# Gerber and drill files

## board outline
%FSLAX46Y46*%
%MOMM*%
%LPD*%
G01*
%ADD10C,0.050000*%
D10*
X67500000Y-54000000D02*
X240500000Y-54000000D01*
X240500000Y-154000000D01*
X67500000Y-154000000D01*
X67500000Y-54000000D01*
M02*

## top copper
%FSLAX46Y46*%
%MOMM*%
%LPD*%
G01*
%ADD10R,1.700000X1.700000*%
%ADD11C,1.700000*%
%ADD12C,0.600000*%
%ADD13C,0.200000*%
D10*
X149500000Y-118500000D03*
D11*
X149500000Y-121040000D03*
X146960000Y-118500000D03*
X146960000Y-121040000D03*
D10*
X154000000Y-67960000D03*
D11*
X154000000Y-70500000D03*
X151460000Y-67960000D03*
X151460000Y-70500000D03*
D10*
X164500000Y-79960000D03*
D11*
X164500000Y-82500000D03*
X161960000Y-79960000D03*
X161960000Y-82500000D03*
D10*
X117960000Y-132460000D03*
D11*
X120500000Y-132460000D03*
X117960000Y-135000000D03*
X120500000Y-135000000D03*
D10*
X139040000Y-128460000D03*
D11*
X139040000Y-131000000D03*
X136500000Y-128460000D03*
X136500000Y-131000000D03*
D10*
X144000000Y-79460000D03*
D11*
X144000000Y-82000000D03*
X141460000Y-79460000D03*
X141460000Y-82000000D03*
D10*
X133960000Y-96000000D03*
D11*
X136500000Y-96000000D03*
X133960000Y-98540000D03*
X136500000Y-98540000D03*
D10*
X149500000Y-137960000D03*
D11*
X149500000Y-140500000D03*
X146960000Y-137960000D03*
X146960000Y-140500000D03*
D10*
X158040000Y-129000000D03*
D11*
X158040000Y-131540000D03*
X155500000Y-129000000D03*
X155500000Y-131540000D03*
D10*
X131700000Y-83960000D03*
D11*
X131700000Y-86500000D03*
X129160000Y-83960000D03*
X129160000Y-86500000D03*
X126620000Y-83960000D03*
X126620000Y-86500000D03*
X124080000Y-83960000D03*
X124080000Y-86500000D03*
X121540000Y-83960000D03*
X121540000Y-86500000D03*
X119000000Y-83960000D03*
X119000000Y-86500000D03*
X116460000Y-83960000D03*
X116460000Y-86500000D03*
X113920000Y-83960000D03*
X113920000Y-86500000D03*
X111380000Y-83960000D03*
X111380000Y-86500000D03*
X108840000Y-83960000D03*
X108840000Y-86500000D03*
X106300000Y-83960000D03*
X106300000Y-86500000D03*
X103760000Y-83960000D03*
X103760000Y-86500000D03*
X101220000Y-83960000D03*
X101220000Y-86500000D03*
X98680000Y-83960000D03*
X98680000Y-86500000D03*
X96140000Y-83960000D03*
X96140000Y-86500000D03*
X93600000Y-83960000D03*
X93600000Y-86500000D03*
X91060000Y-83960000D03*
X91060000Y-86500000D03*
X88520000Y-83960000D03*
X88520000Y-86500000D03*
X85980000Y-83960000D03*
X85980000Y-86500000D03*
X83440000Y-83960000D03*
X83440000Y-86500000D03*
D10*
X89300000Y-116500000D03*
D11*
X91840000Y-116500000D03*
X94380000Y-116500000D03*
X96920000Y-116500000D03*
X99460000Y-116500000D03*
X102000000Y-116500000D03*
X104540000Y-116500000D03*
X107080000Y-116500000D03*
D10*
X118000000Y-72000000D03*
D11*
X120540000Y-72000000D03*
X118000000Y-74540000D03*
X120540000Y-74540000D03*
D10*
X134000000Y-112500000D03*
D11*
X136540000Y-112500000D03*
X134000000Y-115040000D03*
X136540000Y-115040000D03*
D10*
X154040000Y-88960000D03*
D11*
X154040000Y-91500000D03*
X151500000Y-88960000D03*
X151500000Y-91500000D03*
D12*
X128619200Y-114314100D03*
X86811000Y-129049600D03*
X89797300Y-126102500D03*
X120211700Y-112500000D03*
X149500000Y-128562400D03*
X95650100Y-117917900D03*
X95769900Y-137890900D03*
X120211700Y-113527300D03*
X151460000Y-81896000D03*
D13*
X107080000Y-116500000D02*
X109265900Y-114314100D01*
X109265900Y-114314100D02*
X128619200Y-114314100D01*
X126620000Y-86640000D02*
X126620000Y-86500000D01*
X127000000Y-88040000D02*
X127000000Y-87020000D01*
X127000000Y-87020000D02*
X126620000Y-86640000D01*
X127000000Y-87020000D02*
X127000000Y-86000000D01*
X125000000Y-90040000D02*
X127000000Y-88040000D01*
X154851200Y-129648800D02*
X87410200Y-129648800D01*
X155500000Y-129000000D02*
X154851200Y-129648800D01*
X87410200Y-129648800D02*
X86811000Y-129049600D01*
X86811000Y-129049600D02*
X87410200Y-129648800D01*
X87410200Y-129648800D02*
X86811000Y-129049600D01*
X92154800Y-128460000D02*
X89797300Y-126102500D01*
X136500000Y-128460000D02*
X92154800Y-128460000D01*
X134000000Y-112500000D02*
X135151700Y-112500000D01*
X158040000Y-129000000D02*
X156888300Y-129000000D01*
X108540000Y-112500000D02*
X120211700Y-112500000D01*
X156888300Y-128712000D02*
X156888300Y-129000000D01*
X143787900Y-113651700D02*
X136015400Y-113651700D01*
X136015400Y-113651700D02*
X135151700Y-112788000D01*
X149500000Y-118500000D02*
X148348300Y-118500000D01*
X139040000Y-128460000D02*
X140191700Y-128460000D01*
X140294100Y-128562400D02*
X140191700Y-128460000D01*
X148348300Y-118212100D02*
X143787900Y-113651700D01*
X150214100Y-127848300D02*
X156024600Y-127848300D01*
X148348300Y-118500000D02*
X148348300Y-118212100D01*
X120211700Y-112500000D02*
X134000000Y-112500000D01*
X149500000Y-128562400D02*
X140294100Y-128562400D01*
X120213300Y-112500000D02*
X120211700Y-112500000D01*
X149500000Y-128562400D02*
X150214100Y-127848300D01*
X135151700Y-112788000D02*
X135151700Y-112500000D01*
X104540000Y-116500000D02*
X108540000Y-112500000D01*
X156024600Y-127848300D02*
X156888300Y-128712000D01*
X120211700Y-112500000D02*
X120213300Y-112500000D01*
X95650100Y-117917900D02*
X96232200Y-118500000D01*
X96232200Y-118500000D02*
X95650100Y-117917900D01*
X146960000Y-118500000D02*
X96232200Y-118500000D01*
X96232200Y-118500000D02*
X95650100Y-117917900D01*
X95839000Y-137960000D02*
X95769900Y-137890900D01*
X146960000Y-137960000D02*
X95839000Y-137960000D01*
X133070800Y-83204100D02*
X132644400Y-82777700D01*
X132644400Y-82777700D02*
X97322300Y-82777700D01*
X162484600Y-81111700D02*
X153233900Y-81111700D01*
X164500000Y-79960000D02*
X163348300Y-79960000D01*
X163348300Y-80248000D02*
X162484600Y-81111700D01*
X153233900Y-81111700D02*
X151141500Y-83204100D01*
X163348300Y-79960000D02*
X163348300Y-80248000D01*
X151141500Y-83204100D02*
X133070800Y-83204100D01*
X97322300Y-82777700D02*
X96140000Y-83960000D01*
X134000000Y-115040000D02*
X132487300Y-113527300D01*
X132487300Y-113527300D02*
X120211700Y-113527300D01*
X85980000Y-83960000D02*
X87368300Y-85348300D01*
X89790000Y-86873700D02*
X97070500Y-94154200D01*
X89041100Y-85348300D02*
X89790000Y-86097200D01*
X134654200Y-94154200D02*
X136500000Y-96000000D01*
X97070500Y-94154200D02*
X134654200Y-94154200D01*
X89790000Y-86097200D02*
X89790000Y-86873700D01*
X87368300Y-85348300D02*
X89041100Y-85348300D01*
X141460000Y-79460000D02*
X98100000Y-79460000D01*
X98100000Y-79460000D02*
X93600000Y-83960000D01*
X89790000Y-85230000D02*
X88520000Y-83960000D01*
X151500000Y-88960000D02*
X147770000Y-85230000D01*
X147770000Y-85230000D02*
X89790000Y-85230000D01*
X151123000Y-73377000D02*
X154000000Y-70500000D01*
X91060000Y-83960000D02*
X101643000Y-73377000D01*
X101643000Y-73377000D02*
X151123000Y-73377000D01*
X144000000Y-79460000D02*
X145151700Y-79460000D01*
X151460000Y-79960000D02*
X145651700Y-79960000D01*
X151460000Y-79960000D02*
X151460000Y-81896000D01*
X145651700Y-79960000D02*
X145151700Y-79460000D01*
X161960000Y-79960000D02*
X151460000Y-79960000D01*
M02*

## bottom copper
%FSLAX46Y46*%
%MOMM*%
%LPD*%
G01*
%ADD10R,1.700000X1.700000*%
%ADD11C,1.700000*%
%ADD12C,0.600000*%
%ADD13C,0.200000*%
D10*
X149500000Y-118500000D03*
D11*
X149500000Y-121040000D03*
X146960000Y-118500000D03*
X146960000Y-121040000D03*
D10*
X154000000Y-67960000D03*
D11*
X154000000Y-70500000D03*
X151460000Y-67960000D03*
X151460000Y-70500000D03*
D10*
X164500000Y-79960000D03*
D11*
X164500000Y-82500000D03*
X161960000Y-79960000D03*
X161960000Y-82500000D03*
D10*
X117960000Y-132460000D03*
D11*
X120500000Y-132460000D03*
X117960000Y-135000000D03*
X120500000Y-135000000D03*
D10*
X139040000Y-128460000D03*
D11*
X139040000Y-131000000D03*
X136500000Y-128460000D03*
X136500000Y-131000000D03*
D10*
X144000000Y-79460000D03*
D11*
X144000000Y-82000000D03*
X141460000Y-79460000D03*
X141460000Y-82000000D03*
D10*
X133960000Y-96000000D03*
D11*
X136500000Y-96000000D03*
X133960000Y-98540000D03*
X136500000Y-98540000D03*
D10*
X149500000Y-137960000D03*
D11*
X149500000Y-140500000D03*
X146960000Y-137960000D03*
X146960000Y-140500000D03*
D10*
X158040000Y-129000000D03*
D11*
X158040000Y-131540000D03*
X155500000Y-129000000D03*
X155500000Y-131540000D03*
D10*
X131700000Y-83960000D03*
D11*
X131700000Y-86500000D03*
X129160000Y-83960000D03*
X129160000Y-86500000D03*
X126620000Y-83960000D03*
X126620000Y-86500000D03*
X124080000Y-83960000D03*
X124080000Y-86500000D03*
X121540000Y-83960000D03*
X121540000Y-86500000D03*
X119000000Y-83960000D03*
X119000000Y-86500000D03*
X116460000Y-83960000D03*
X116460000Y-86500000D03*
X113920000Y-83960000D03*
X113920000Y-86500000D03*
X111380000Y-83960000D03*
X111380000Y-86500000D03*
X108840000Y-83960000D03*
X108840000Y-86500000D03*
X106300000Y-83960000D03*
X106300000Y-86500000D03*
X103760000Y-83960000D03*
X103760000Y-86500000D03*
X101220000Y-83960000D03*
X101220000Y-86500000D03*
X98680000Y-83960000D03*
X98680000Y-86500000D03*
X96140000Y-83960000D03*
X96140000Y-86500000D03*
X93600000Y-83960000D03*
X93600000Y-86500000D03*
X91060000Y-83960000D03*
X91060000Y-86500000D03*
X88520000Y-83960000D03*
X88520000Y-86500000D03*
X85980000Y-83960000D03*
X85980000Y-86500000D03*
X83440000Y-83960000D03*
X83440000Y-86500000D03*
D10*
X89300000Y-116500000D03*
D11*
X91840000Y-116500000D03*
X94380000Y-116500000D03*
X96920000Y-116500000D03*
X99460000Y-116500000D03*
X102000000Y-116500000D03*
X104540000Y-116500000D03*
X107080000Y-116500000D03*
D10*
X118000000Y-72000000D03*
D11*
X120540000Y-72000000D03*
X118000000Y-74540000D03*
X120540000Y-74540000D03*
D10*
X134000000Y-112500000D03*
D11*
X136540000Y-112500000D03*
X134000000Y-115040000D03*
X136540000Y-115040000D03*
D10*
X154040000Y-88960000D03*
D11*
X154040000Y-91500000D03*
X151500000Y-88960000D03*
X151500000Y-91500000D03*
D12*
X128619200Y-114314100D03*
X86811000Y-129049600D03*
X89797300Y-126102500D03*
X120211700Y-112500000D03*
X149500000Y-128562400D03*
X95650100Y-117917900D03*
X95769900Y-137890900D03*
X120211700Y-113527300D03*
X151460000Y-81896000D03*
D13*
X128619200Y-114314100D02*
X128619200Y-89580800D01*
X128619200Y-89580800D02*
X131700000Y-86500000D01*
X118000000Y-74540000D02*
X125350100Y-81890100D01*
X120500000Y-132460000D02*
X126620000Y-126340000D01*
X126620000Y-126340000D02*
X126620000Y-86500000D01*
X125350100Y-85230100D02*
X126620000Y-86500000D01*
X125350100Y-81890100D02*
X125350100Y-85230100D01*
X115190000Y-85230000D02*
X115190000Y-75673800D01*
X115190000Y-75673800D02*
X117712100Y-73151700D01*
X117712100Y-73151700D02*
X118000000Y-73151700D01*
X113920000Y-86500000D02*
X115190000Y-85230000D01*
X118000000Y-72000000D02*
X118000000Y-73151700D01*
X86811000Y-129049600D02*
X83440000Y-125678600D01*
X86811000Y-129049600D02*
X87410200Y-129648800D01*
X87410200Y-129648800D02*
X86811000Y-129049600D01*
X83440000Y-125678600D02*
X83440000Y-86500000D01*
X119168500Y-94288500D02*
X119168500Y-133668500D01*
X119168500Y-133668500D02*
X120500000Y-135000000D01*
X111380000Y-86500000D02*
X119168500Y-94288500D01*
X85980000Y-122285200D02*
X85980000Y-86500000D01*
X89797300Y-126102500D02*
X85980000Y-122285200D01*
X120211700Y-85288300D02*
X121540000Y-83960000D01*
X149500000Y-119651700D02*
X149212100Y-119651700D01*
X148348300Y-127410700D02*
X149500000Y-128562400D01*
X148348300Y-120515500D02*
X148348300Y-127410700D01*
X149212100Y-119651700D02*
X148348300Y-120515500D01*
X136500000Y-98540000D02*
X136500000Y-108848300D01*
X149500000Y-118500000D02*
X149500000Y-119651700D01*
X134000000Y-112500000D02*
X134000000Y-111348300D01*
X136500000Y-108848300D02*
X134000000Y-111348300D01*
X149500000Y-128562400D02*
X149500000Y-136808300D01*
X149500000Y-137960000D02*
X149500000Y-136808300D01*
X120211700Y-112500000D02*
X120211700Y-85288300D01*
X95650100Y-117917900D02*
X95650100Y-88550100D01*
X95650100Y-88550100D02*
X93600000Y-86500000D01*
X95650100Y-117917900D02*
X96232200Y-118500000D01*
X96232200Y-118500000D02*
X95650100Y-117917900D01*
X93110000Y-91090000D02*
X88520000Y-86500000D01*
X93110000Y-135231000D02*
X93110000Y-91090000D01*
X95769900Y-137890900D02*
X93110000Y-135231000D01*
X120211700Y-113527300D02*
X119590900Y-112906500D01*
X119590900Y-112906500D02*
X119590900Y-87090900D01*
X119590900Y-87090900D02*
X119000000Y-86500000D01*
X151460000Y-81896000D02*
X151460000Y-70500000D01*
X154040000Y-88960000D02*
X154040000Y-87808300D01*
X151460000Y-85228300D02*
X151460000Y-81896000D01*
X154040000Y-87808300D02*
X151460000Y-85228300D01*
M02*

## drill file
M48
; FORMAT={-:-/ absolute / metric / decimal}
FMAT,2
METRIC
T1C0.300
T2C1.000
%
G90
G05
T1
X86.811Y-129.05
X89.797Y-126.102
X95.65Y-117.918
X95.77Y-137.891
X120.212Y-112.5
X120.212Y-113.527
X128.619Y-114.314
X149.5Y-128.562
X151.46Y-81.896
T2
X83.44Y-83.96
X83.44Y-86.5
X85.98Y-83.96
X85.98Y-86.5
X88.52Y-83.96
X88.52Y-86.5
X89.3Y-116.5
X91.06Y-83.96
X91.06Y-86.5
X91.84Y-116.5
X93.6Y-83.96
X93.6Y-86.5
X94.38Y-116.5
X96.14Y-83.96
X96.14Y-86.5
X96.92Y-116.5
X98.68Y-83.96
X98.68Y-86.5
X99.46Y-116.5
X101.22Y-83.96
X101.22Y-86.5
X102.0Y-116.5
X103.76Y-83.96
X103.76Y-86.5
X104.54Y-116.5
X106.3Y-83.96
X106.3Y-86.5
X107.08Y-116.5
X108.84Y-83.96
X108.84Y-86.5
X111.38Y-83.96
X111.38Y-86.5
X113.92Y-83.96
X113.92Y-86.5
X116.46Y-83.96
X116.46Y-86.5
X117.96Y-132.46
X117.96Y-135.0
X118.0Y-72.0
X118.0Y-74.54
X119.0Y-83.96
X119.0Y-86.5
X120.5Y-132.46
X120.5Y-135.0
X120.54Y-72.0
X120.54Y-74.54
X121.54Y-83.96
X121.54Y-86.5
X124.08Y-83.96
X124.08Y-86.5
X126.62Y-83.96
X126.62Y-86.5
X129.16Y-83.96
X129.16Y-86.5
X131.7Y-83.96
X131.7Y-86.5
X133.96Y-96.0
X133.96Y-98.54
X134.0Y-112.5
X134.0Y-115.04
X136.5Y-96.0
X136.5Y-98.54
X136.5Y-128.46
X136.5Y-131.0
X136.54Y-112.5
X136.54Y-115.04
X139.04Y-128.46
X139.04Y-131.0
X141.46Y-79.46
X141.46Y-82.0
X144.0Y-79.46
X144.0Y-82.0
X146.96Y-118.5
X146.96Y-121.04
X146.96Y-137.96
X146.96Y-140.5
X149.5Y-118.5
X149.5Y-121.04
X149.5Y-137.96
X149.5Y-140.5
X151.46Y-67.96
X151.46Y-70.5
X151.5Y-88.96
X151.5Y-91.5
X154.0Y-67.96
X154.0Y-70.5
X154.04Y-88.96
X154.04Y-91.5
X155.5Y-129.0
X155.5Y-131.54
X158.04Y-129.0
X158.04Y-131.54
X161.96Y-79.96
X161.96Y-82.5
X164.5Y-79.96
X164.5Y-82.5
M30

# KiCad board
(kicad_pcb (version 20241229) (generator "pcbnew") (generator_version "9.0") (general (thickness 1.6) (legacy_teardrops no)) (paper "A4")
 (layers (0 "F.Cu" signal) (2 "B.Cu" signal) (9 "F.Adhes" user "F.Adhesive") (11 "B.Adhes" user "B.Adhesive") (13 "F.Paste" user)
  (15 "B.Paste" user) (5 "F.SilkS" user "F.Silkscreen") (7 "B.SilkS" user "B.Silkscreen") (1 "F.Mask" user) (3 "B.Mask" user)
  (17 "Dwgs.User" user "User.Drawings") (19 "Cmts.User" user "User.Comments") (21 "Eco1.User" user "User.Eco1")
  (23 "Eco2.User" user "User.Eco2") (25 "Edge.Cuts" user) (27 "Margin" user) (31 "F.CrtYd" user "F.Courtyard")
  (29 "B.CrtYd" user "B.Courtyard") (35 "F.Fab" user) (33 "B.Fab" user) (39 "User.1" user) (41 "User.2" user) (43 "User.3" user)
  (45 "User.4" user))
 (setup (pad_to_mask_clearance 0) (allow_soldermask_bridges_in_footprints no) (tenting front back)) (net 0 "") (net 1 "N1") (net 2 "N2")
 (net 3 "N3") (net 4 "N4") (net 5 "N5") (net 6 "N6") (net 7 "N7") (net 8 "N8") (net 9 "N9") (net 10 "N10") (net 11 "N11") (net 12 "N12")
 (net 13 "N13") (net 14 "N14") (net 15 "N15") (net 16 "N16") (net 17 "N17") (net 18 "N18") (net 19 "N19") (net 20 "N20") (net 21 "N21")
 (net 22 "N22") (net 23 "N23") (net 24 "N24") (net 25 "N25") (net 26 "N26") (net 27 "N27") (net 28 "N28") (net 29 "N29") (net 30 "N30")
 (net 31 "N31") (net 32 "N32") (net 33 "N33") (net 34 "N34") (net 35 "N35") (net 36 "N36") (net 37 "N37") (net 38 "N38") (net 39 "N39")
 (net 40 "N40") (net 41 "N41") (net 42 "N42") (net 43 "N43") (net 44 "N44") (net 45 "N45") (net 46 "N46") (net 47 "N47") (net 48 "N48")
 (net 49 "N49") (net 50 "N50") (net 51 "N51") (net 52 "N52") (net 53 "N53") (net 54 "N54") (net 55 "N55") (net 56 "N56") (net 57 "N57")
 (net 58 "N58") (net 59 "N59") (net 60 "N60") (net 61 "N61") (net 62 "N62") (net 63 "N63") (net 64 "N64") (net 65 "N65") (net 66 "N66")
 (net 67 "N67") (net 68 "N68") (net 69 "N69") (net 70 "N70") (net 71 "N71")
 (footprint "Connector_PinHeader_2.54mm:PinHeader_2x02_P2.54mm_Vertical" (layer "F.Cu") (at 149.5 118.5 -90)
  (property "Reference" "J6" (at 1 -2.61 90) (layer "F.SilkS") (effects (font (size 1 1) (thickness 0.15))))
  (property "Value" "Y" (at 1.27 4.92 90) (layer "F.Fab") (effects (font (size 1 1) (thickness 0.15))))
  (pad "1" thru_hole rect (at 0 0 270) (size 1.7 1.7) (drill 1) (layers "*.Cu" "*.Mask") (remove_unused_layers no) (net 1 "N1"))
  (pad "2" thru_hole circle (at 2.54 0 270) (size 1.7 1.7) (drill 1) (layers "*.Cu" "*.Mask") (remove_unused_layers no) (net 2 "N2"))
  (pad "3" thru_hole circle (at 0 2.54 270) (size 1.7 1.7) (drill 1) (layers "*.Cu" "*.Mask") (remove_unused_layers no) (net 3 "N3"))
  (pad "4" thru_hole circle (at 2.54 2.54 270) (size 1.7 1.7) (drill 1) (layers "*.Cu" "*.Mask") (remove_unused_layers no) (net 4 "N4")))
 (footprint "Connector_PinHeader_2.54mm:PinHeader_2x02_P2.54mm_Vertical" (layer "F.Cu") (at 154 67.96 -90)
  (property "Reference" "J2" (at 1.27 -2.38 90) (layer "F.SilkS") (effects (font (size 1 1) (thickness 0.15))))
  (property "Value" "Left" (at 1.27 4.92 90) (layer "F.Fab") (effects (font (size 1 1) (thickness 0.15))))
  (pad "1" thru_hole rect (at 0 0 270) (size 1.7 1.7) (drill 1) (layers "*.Cu" "*.Mask") (remove_unused_layers no) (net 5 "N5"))
  (pad "2" thru_hole circle (at 2.54 0 270) (size 1.7 1.7) (drill 1) (layers "*.Cu" "*.Mask") (remove_unused_layers no) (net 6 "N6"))
  (pad "3" thru_hole circle (at 0 2.54 270) (size 1.7 1.7) (drill 1) (layers "*.Cu" "*.Mask") (remove_unused_layers no) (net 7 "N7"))
  (pad "4" thru_hole circle (at 2.54 2.54 270) (size 1.7 1.7) (drill 1) (layers "*.Cu" "*.Mask") (remove_unused_layers no) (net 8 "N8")))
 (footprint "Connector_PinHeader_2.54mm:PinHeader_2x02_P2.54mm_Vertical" (layer "F.Cu") (at 164.5 79.96 -90)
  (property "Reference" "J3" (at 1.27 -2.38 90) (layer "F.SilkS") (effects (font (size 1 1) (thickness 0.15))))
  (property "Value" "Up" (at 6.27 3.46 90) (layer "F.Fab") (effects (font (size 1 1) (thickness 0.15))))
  (pad "1" thru_hole rect (at 0 0 270) (size 1.7 1.7) (drill 1) (layers "*.Cu" "*.Mask") (remove_unused_layers no) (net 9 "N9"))
  (pad "2" thru_hole circle (at 2.54 0 270) (size 1.7 1.7) (drill 1) (layers "*.Cu" "*.Mask") (remove_unused_layers no) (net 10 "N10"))
  (pad "3" thru_hole circle (at 0 2.54 270) (size 1.7 1.7) (drill 1) (layers "*.Cu" "*.Mask") (remove_unused_layers no) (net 8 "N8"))
  (pad "4" thru_hole circle (at 2.54 2.54 270) (size 1.7 1.7) (drill 1) (layers "*.Cu" "*.Mask") (remove_unused_layers no) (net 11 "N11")))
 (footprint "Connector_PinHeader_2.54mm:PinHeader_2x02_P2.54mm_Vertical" (layer "F.Cu") (at 117.96 132.46)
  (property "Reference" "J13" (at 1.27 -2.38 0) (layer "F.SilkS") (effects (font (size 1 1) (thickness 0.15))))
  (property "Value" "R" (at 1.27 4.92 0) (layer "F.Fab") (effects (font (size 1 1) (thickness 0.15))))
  (pad "1" thru_hole rect (at 0 0) (size 1.7 1.7) (drill 1) (layers "*.Cu" "*.Mask") (remove_unused_layers no) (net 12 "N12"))
  (pad "2" thru_hole circle (at 2.54 0) (size 1.7 1.7) (drill 1) (layers "*.Cu" "*.Mask") (remove_unused_layers no) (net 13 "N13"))
  (pad "3" thru_hole circle (at 0 2.54) (size 1.7 1.7) (drill 1) (layers "*.Cu" "*.Mask") (remove_unused_layers no) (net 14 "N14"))
  (pad "4" thru_hole circle (at 2.54 2.54) (size 1.7 1.7) (drill 1) (layers "*.Cu" "*.Mask") (remove_unused_layers no) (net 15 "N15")))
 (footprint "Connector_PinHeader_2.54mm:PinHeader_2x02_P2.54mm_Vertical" (layer "F.Cu") (at 139.04 128.46 -90)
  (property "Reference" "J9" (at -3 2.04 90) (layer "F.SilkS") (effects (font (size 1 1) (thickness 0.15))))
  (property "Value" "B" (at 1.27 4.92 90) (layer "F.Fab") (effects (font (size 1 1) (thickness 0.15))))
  (pad "1" thru_hole rect (at 0 0 270) (size 1.7 1.7) (drill 1) (layers "*.Cu" "*.Mask") (remove_unused_layers no) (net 1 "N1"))
  (pad "2" thru_hole circle (at 2.54 0 270) (size 1.7 1.7) (drill 1) (layers "*.Cu" "*.Mask") (remove_unused_layers no) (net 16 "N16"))
  (pad "3" thru_hole circle (at 0 2.54 270) (size 1.7 1.7) (drill 1) (layers "*.Cu" "*.Mask") (remove_unused_layers no) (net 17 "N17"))
  (pad "4" thru_hole circle (at 2.54 2.54 270) (size 1.7 1.7) (drill 1) (layers "*.Cu" "*.Mask") (remove_unused_layers no) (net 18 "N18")))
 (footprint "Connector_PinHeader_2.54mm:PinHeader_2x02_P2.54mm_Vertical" (layer "F.Cu") (at 144 79.46 -90)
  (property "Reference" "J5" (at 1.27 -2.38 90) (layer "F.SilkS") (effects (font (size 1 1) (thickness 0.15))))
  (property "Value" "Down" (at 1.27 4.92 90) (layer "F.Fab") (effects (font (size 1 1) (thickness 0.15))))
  (pad "1" thru_hole rect (at 0 0 270) (size 1.7 1.7) (drill 1) (layers "*.Cu" "*.Mask") (remove_unused_layers no) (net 8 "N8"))
  (pad "2" thru_hole circle (at 2.54 0 270) (size 1.7 1.7) (drill 1) (layers "*.Cu" "*.Mask") (remove_unused_layers no) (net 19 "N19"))
  (pad "3" thru_hole circle (at 0 2.54 270) (size 1.7 1.7) (drill 1) (layers "*.Cu" "*.Mask") (remove_unused_layers no) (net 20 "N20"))
  (pad "4" thru_hole circle (at 2.54 2.54 270) (size 1.7 1.7) (drill 1) (layers "*.Cu" "*.Mask") (remove_unused_layers no) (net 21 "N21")))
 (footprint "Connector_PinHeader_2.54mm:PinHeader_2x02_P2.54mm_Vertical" (layer "F.Cu") (at 133.96 96)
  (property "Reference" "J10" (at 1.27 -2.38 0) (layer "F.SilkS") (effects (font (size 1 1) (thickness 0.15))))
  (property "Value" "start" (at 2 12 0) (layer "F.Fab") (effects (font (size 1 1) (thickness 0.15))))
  (pad "1" thru_hole rect (at 0 0) (size 1.7 1.7) (drill 1) (layers "*.Cu" "*.Mask") (remove_unused_layers no) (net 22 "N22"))
  (pad "2" thru_hole circle (at 2.54 0) (size 1.7 1.7) (drill 1) (layers "*.Cu" "*.Mask") (remove_unused_layers no) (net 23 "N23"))
  (pad "3" thru_hole circle (at 0 2.54) (size 1.7 1.7) (drill 1) (layers "*.Cu" "*.Mask") (remove_unused_layers no) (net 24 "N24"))
  (pad "4" thru_hole circle (at 2.54 2.54) (size 1.7 1.7) (drill 1) (layers "*.Cu" "*.Mask") (remove_unused_layers no) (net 1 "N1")))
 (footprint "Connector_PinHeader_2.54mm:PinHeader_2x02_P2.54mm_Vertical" (layer "F.Cu") (at 149.5 137.96 -90)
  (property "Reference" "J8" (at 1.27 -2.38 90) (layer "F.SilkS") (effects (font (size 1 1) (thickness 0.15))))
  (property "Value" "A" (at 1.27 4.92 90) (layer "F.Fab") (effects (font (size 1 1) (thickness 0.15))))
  (pad "1" thru_hole rect (at 0 0 270) (size 1.7 1.7) (drill 1) (layers "*.Cu" "*.Mask") (remove_unused_layers no) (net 1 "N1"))
  (pad "2" thru_hole circle (at 2.54 0 270) (size 1.7 1.7) (drill 1) (layers "*.Cu" "*.Mask") (remove_unused_layers no) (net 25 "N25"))
  (pad "3" thru_hole circle (at 0 2.54 270) (size 1.7 1.7) (drill 1) (layers "*.Cu" "*.Mask") (remove_unused_layers no) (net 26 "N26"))
  (pad "4" thru_hole circle (at 2.54 2.54 270) (size 1.7 1.7) (drill 1) (layers "*.Cu" "*.Mask") (remove_unused_layers no) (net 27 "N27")))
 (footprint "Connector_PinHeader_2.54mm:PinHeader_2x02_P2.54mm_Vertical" (layer "F.Cu") (at 158.04 129 -90)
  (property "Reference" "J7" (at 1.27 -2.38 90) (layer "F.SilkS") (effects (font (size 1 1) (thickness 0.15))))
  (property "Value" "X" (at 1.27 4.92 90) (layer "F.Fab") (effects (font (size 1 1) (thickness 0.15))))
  (pad "1" thru_hole rect (at 0 0 270) (size 1.7 1.7) (drill 1) (layers "*.Cu" "*.Mask") (remove_unused_layers no) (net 1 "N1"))
  (pad "2" thru_hole circle (at 2.54 0 270) (size 1.7 1.7) (drill 1) (layers "*.Cu" "*.Mask") (remove_unused_layers no) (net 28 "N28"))
  (pad "3" thru_hole circle (at 0 2.54 270) (size 1.7 1.7) (drill 1) (layers "*.Cu" "*.Mask") (remove_unused_layers no) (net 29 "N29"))
  (pad "4" thru_hole circle (at 2.54 2.54 270) (size 1.7 1.7) (drill 1) (layers "*.Cu" "*.Mask") (remove_unused_layers no) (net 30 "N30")))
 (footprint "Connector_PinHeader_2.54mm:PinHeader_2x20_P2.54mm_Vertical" (layer "F.Cu") (at 131.7 83.96 -90)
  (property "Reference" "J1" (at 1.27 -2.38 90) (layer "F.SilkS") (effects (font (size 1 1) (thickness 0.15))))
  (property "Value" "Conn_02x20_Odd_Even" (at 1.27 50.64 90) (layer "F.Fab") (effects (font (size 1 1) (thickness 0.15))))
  (pad "1" thru_hole rect (at 0 0 270) (size 1.7 1.7) (drill 1) (layers "*.Cu" "*.Mask") (remove_unused_layers no) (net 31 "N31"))
  (pad "2" thru_hole circle (at 2.54 0 270) (size 1.7 1.7) (drill 1) (layers "*.Cu" "*.Mask") (remove_unused_layers no) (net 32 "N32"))
  (pad "3" thru_hole circle (at 0 2.54 270) (size 1.7 1.7) (drill 1) (layers "*.Cu" "*.Mask") (remove_unused_layers no) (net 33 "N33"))
  (pad "4" thru_hole circle (at 2.54 2.54 270) (size 1.7 1.7) (drill 1) (layers "*.Cu" "*.Mask") (remove_unused_layers no) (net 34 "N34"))
  (pad "5" thru_hole circle (at 0 5.08 270) (size 1.7 1.7) (drill 1) (layers "*.Cu" "*.Mask") (remove_unused_layers no) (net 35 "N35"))
  (pad "6" thru_hole circle (at 2.54 5.08 270) (size 1.7 1.7) (drill 1) (layers "*.Cu" "*.Mask") (remove_unused_layers no) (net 13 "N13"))
  (pad "7" thru_hole circle (at 0 7.62 270) (size 1.7 1.7) (drill 1) (layers "*.Cu" "*.Mask") (remove_unused_layers no) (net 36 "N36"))
  (pad "8" thru_hole circle (at 2.54 7.62 270) (size 1.7 1.7) (drill 1) (layers "*.Cu" "*.Mask") (remove_unused_layers no) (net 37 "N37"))
  (pad "9" thru_hole circle (at 0 10.16 270) (size 1.7 1.7) (drill 1) (layers "*.Cu" "*.Mask") (remove_unused_layers no) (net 1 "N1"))
  (pad "10" thru_hole circle (at 2.54 10.16 270) (size 1.7 1.7) (drill 1) (layers "*.Cu" "*.Mask") (remove_unused_layers no) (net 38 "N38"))
  (pad "11" thru_hole circle (at 0 12.7 270) (size 1.7 1.7) (drill 1) (layers "*.Cu" "*.Mask") (remove_unused_layers no) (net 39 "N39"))
  (pad "12" thru_hole circle (at 2.54 12.7 270) (size 1.7 1.7) (drill 1) (layers "*.Cu" "*.Mask") (remove_unused_layers no) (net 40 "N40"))
  (pad "13" thru_hole circle (at 0 15.24 270) (size 1.7 1.7) (drill 1) (layers "*.Cu" "*.Mask") (remove_unused_layers no) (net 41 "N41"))
  (pad "14" thru_hole circle (at 2.54 15.24 270) (size 1.7 1.7) (drill 1) (layers "*.Cu" "*.Mask") (remove_unused_layers no) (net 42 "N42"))
  (pad "15" thru_hole circle (at 0 17.78 270) (size 1.7 1.7) (drill 1) (layers "*.Cu" "*.Mask") (remove_unused_layers no) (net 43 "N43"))
  (pad "16" thru_hole circle (at 2.54 17.78 270) (size 1.7 1.7) (drill 1) (layers "*.Cu" "*.Mask") (remove_unused_layers no) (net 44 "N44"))
  (pad "17" thru_hole circle (at 0 20.32 270) (size 1.7 1.7) (drill 1) (layers "*.Cu" "*.Mask") (remove_unused_layers no) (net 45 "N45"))
  (pad "18" thru_hole circle (at 2.54 20.32 270) (size 1.7 1.7) (drill 1) (layers "*.Cu" "*.Mask") (remove_unused_layers no) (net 15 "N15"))
  (pad "19" thru_hole circle (at 0 22.86 270) (size 1.7 1.7) (drill 1) (layers "*.Cu" "*.Mask") (remove_unused_layers no) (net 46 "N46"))
  (pad "20" thru_hole circle (at 2.54 22.86 270) (size 1.7 1.7) (drill 1) (layers "*.Cu" "*.Mask") (remove_unused_layers no) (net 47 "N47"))
  (pad "21" thru_hole circle (at 0 25.4 270) (size 1.7 1.7) (drill 1) (layers "*.Cu" "*.Mask") (remove_unused_layers no) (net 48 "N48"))
  (pad "22" thru_hole circle (at 2.54 25.4 270) (size 1.7 1.7) (drill 1) (layers "*.Cu" "*.Mask") (remove_unused_layers no) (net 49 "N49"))
  (pad "23" thru_hole circle (at 0 27.94 270) (size 1.7 1.7) (drill 1) (layers "*.Cu" "*.Mask") (remove_unused_layers no) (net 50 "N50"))
  (pad "24" thru_hole circle (at 2.54 27.94 270) (size 1.7 1.7) (drill 1) (layers "*.Cu" "*.Mask") (remove_unused_layers no) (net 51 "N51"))
  (pad "25" thru_hole circle (at 0 30.48 270) (size 1.7 1.7) (drill 1) (layers "*.Cu" "*.Mask") (remove_unused_layers no) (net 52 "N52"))
  (pad "26" thru_hole circle (at 2.54 30.48 270) (size 1.7 1.7) (drill 1) (layers "*.Cu" "*.Mask") (remove_unused_layers no) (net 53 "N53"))
  (pad "27" thru_hole circle (at 0 33.02 270) (size 1.7 1.7) (drill 1) (layers "*.Cu" "*.Mask") (remove_unused_layers no) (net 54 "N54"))
  (pad "28" thru_hole circle (at 2.54 33.02 270) (size 1.7 1.7) (drill 1) (layers "*.Cu" "*.Mask") (remove_unused_layers no) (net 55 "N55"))
  (pad "29" thru_hole circle (at 0 35.56 270) (size 1.7 1.7) (drill 1) (layers "*.Cu" "*.Mask") (remove_unused_layers no) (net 9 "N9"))
  (pad "30" thru_hole circle (at 2.54 35.56 270) (size 1.7 1.7) (drill 1) (layers "*.Cu" "*.Mask") (remove_unused_layers no) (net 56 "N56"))
  (pad "31" thru_hole circle (at 0 38.1 270) (size 1.7 1.7) (drill 1) (layers "*.Cu" "*.Mask") (remove_unused_layers no) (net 20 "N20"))
  (pad "32" thru_hole circle (at 2.54 38.1 270) (size 1.7 1.7) (drill 1) (layers "*.Cu" "*.Mask") (remove_unused_layers no) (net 3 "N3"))
  (pad "33" thru_hole circle (at 0 40.64 270) (size 1.7 1.7) (drill 1) (layers "*.Cu" "*.Mask") (remove_unused_layers no) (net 6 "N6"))
  (pad "34" thru_hole circle (at 2.54 40.64 270) (size 1.7 1.7) (drill 1) (layers "*.Cu" "*.Mask") (remove_unused_layers no) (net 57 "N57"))
  (pad "35" thru_hole circle (at 0 43.18 270) (size 1.7 1.7) (drill 1) (layers "*.Cu" "*.Mask") (remove_unused_layers no) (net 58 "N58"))
  (pad "36" thru_hole circle (at 2.54 43.18 270) (size 1.7 1.7) (drill 1) (layers "*.Cu" "*.Mask") (remove_unused_layers no) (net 26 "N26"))
  (pad "37" thru_hole circle (at 0 45.72 270) (size 1.7 1.7) (drill 1) (layers "*.Cu" "*.Mask") (remove_unused_layers no) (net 23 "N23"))
  (pad "38" thru_hole circle (at 2.54 45.72 270) (size 1.7 1.7) (drill 1) (layers "*.Cu" "*.Mask") (remove_unused_layers no) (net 17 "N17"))
  (pad "39" thru_hole circle (at 0 48.26 270) (size 1.7 1.7) (drill 1) (layers "*.Cu" "*.Mask") (remove_unused_layers no) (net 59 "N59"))
  (pad "40" thru_hole circle (at 2.54 48.26 270) (size 1.7 1.7) (drill 1) (layers "*.Cu" "*.Mask") (remove_unused_layers no) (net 29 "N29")))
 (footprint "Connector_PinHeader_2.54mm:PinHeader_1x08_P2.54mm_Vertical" (layer "F.Cu") (at 89.3 116.5 90)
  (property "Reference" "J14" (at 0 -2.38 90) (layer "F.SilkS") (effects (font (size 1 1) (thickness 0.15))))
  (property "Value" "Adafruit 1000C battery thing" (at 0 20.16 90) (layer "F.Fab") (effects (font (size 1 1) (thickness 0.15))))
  (pad "1" thru_hole rect (at 0 0 90) (size 1.7 1.7) (drill 1) (layers "*.Cu" "*.Mask") (remove_unused_layers no) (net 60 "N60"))
  (pad "2" thru_hole circle (at 0 2.54 90) (size 1.7 1.7) (drill 1) (layers "*.Cu" "*.Mask") (remove_unused_layers no) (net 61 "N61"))
  (pad "3" thru_hole circle (at 0 5.08 90) (size 1.7 1.7) (drill 1) (layers "*.Cu" "*.Mask") (remove_unused_layers no) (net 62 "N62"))
  (pad "4" thru_hole circle (at 0 7.62 90) (size 1.7 1.7) (drill 1) (layers "*.Cu" "*.Mask") (remove_unused_layers no) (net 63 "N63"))
  (pad "5" thru_hole circle (at 0 10.16 90) (size 1.7 1.7) (drill 1) (layers "*.Cu" "*.Mask") (remove_unused_layers no) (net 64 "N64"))
  (pad "6" thru_hole circle (at 0 12.7 90) (size 1.7 1.7) (drill 1) (layers "*.Cu" "*.Mask") (remove_unused_layers no) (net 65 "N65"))
  (pad "7" thru_hole circle (at 0 15.24 90) (size 1.7 1.7) (drill 1) (layers "*.Cu" "*.Mask") (remove_unused_layers no) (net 1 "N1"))
  (pad "8" thru_hole circle (at 0 17.78 90) (size 1.7 1.7) (drill 1) (layers "*.Cu" "*.Mask") (remove_unused_layers no) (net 32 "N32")))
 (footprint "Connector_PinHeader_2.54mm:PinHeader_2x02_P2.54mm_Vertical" (layer "F.Cu") (at 118 72)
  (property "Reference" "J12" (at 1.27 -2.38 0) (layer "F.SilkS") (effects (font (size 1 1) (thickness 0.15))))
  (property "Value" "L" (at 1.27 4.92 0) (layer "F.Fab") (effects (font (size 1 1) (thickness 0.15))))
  (pad "1" thru_hole rect (at 0 0) (size 1.7 1.7) (drill 1) (layers "*.Cu" "*.Mask") (remove_unused_layers no) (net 44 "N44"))
  (pad "2" thru_hole circle (at 2.54 0) (size 1.7 1.7) (drill 1) (layers "*.Cu" "*.Mask") (remove_unused_layers no) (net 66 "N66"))
  (pad "3" thru_hole circle (at 0 2.54) (size 1.7 1.7) (drill 1) (layers "*.Cu" "*.Mask") (remove_unused_layers no) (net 13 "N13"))
  (pad "4" thru_hole circle (at 2.54 2.54) (size 1.7 1.7) (drill 1) (layers "*.Cu" "*.Mask") (remove_unused_layers no) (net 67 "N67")))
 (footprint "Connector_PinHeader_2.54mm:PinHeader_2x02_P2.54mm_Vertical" (layer "F.Cu") (at 134 112.5)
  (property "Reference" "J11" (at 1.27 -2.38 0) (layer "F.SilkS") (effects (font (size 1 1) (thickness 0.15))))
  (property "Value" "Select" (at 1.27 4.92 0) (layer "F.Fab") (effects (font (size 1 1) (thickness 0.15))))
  (pad "1" thru_hole rect (at 0 0) (size 1.7 1.7) (drill 1) (layers "*.Cu" "*.Mask") (remove_unused_layers no) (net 1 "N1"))
  (pad "2" thru_hole circle (at 2.54 0) (size 1.7 1.7) (drill 1) (layers "*.Cu" "*.Mask") (remove_unused_layers no) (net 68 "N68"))
  (pad "3" thru_hole circle (at 0 2.54) (size 1.7 1.7) (drill 1) (layers "*.Cu" "*.Mask") (remove_unused_layers no) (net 40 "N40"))
  (pad "4" thru_hole circle (at 2.54 2.54) (size 1.7 1.7) (drill 1) (layers "*.Cu" "*.Mask") (remove_unused_layers no) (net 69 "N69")))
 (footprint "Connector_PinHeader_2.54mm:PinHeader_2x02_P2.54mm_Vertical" (layer "F.Cu") (at 154.04 88.96 -90)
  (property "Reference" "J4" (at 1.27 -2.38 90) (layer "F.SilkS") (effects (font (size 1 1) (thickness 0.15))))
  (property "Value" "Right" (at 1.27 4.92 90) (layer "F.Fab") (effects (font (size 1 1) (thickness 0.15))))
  (pad "1" thru_hole rect (at 0 0 270) (size 1.7 1.7) (drill 1) (layers "*.Cu" "*.Mask") (remove_unused_layers no) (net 8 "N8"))
  (pad "2" thru_hole circle (at 2.54 0 270) (size 1.7 1.7) (drill 1) (layers "*.Cu" "*.Mask") (remove_unused_layers no) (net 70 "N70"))
  (pad "3" thru_hole circle (at 0 2.54 270) (size 1.7 1.7) (drill 1) (layers "*.Cu" "*.Mask") (remove_unused_layers no) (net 58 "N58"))
  (pad "4" thru_hole circle (at 2.54 2.54 270) (size 1.7 1.7) (drill 1) (layers "*.Cu" "*.Mask") (remove_unused_layers no) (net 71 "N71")))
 (gr_rect (start 67.5 54) (end 240.5 154) (stroke (width 0.05) (type default)) (fill no) (layer "Edge.Cuts"))
 (segment (start 107.08 116.5) (end 109.2659 114.3141) (width 0.2) (layer "F.Cu") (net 32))
 (segment (start 109.2659 114.3141) (end 128.6192 114.3141) (width 0.2) (layer "F.Cu") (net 32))
 (via (at 128.6192 114.3141) (size 0.6) (drill 0.3) (layers "F.Cu" "B.Cu") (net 32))
 (segment (start 128.6192 114.3141) (end 128.6192 89.5808) (width 0.2) (layer "B.Cu") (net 32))
 (segment (start 128.6192 89.5808) (end 131.7 86.5) (width 0.2) (layer "B.Cu") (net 32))
 (segment (start 126.62 86.64) (end 126.62 86.5) (width 0.2) (layer "F.Cu") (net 13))
 (segment (start 127 88.04) (end 127 87.02) (width 0.2) (layer "F.Cu") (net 13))
 (segment (start 127 87.02) (end 126.62 86.64) (width 0.2) (layer "F.Cu") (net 13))
 (segment (start 127 87.02) (end 127 86) (width 0.2) (layer "F.Cu") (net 13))
 (segment (start 125 90.04) (end 127 88.04) (width 0.2) (layer "F.Cu") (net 13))
 (segment (start 118 74.54) (end 125.3501 81.8901) (width 0.2) (layer "B.Cu") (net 13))
 (segment (start 120.5 132.46) (end 126.62 126.34) (width 0.2) (layer "B.Cu") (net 13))
 (segment (start 126.62 126.34) (end 126.62 86.5) (width 0.2) (layer "B.Cu") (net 13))
 (segment (start 125.3501 85.2301) (end 126.62 86.5) (width 0.2) (layer "B.Cu") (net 13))
 (segment (start 125.3501 81.8901) (end 125.3501 85.2301) (width 0.2) (layer "B.Cu") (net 13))
 (segment (start 115.19 85.23) (end 115.19 75.6738) (width 0.2) (layer "B.Cu") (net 44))
 (segment (start 115.19 75.6738) (end 117.7121 73.1517) (width 0.2) (layer "B.Cu") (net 44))
 (segment (start 117.7121 73.1517) (end 118 73.1517) (width 0.2) (layer "B.Cu") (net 44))
 (segment (start 113.92 86.5) (end 115.19 85.23) (width 0.2) (layer "B.Cu") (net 44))
 (segment (start 118 72) (end 118 73.1517) (width 0.2) (layer "B.Cu") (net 44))
 (segment (start 154.8512 129.6488) (end 87.4102 129.6488) (width 0.2) (layer "F.Cu") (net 29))
 (segment (start 155.5 129) (end 154.8512 129.6488) (width 0.2) (layer "F.Cu") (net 29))
 (segment (start 87.4102 129.6488) (end 86.811 129.0496) (width 0.2) (layer "F.Cu") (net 29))
 (segment (start 86.811 129.0496) (end 87.4102 129.6488) (width 0.2) (layer "F.Cu") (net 29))
 (segment (start 87.4102 129.6488) (end 86.811 129.0496) (width 0.2) (layer "F.Cu") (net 29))
 (via (at 86.811 129.0496) (size 0.6) (drill 0.3) (layers "F.Cu" "B.Cu") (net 29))
 (segment (start 86.811 129.0496) (end 83.44 125.6786) (width 0.2) (layer "B.Cu") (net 29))
 (segment (start 86.811 129.0496) (end 87.4102 129.6488) (width 0.2) (layer "B.Cu") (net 29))
 (segment (start 87.4102 129.6488) (end 86.811 129.0496) (width 0.2) (layer "B.Cu") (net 29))
 (segment (start 83.44 125.6786) (end 83.44 86.5) (width 0.2) (layer "B.Cu") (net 29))
 (segment (start 119.1685 94.2885) (end 119.1685 133.6685) (width 0.2) (layer "B.Cu") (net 15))
 (segment (start 119.1685 133.6685) (end 120.5 135) (width 0.2) (layer "B.Cu") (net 15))
 (segment (start 111.38 86.5) (end 119.1685 94.2885) (width 0.2) (layer "B.Cu") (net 15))
 (segment (start 92.1548 128.46) (end 89.7973 126.1025) (width 0.2) (layer "F.Cu") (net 17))
 (segment (start 136.5 128.46) (end 92.1548 128.46) (width 0.2) (layer "F.Cu") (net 17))
 (via (at 89.7973 126.1025) (size 0.6) (drill 0.3) (layers "F.Cu" "B.Cu") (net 17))
 (segment (start 85.98 122.2852) (end 85.98 86.5) (width 0.2) (layer "B.Cu") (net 17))
 (segment (start 89.7973 126.1025) (end 85.98 122.2852) (width 0.2) (layer "B.Cu") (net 17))
 (segment (start 134 112.5) (end 135.1517 112.5) (width 0.2) (layer "F.Cu") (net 1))
 (segment (start 158.04 129) (end 156.8883 129) (width 0.2) (layer "F.Cu") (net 1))
 (segment (start 108.54 112.5) (end 120.2117 112.5) (width 0.2) (layer "F.Cu") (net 1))
 (segment (start 156.8883 128.712) (end 156.8883 129) (width 0.2) (layer "F.Cu") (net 1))
 (segment (start 143.7879 113.6517) (end 136.0154 113.6517) (width 0.2) (layer "F.Cu") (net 1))
 (segment (start 136.0154 113.6517) (end 135.1517 112.788) (width 0.2) (layer "F.Cu") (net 1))
 (segment (start 149.5 118.5) (end 148.3483 118.5) (width 0.2) (layer "F.Cu") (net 1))
 (segment (start 139.04 128.46) (end 140.1917 128.46) (width 0.2) (layer "F.Cu") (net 1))
 (segment (start 140.2941 128.5624) (end 140.1917 128.46) (width 0.2) (layer "F.Cu") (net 1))
 (segment (start 148.3483 118.2121) (end 143.7879 113.6517) (width 0.2) (layer "F.Cu") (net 1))
 (segment (start 150.2141 127.8483) (end 156.0246 127.8483) (width 0.2) (layer "F.Cu") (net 1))
 (segment (start 148.3483 118.5) (end 148.3483 118.2121) (width 0.2) (layer "F.Cu") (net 1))
 (segment (start 120.2117 112.5) (end 134 112.5) (width 0.2) (layer "F.Cu") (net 1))
 (segment (start 149.5 128.5624) (end 140.2941 128.5624) (width 0.2) (layer "F.Cu") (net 1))
 (segment (start 120.2133 112.5) (end 120.2117 112.5) (width 0.2) (layer "F.Cu") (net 1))
 (segment (start 149.5 128.5624) (end 150.2141 127.8483) (width 0.2) (layer "F.Cu") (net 1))
 (segment (start 135.1517 112.788) (end 135.1517 112.5) (width 0.2) (layer "F.Cu") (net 1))
 (segment (start 104.54 116.5) (end 108.54 112.5) (width 0.2) (layer "F.Cu") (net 1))
 (segment (start 156.0246 127.8483) (end 156.8883 128.712) (width 0.2) (layer "F.Cu") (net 1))
 (segment (start 120.2117 112.5) (end 120.2133 112.5) (width 0.2) (layer "F.Cu") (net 1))
 (via (at 120.2117 112.5) (size 0.6) (drill 0.3) (layers "F.Cu" "B.Cu") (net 1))
 (via (at 149.5 128.5624) (size 0.6) (drill 0.3) (layers "F.Cu" "B.Cu") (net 1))
 (segment (start 120.2117 85.2883) (end 121.54 83.96) (width 0.2) (layer "B.Cu") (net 1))
 (segment (start 149.5 119.6517) (end 149.2121 119.6517) (width 0.2) (layer "B.Cu") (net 1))
 (segment (start 148.3483 127.4107) (end 149.5 128.5624) (width 0.2) (layer "B.Cu") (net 1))
 (segment (start 148.3483 120.5155) (end 148.3483 127.4107) (width 0.2) (layer "B.Cu") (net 1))
 (segment (start 149.2121 119.6517) (end 148.3483 120.5155) (width 0.2) (layer "B.Cu") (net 1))
 (segment (start 136.5 98.54) (end 136.5 108.8483) (width 0.2) (layer "B.Cu") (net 1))
 (segment (start 149.5 118.5) (end 149.5 119.6517) (width 0.2) (layer "B.Cu") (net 1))
 (segment (start 134 112.5) (end 134 111.3483) (width 0.2) (layer "B.Cu") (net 1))
 (segment (start 136.5 108.8483) (end 134 111.3483) (width 0.2) (layer "B.Cu") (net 1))
 (segment (start 149.5 128.5624) (end 149.5 136.8083) (width 0.2) (layer "B.Cu") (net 1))
 (segment (start 149.5 137.96) (end 149.5 136.8083) (width 0.2) (layer "B.Cu") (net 1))
 (segment (start 120.2117 112.5) (end 120.2117 85.2883) (width 0.2) (layer "B.Cu") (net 1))
 (segment (start 95.6501 117.9179) (end 96.2322 118.5) (width 0.2) (layer "F.Cu") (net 3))
 (segment (start 96.2322 118.5) (end 95.6501 117.9179) (width 0.2) (layer "F.Cu") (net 3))
 (segment (start 146.96 118.5) (end 96.2322 118.5) (width 0.2) (layer "F.Cu") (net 3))
 (segment (start 96.2322 118.5) (end 95.6501 117.9179) (width 0.2) (layer "F.Cu") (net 3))
 (via (at 95.6501 117.9179) (size 0.6) (drill 0.3) (layers "F.Cu" "B.Cu") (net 3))
 (segment (start 95.6501 117.9179) (end 95.6501 88.5501) (width 0.2) (layer "B.Cu") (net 3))
 (segment (start 95.6501 88.5501) (end 93.6 86.5) (width 0.2) (layer "B.Cu") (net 3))
 (segment (start 95.6501 117.9179) (end 96.2322 118.5) (width 0.2) (layer "B.Cu") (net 3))
 (segment (start 96.2322 118.5) (end 95.6501 117.9179) (width 0.2) (layer "B.Cu") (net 3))
 (segment (start 95.839 137.96) (end 95.7699 137.8909) (width 0.2) (layer "F.Cu") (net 26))
 (segment (start 146.96 137.96) (end 95.839 137.96) (width 0.2) (layer "F.Cu") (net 26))
 (via (at 95.7699 137.8909) (size 0.6) (drill 0.3) (layers "F.Cu" "B.Cu") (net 26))
 (segment (start 93.11 91.09) (end 88.52 86.5) (width 0.2) (layer "B.Cu") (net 26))
 (segment (start 93.11 135.231) (end 93.11 91.09) (width 0.2) (layer "B.Cu") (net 26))
 (segment (start 95.7699 137.8909) (end 93.11 135.231) (width 0.2) (layer "B.Cu") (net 26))
 (segment (start 133.0708 83.2041) (end 132.6444 82.7777) (width 0.2) (layer "F.Cu") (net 9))
 (segment (start 132.6444 82.7777) (end 97.3223 82.7777) (width 0.2) (layer "F.Cu") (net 9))
 (segment (start 162.4846 81.1117) (end 153.2339 81.1117) (width 0.2) (layer "F.Cu") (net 9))
 (segment (start 164.5 79.96) (end 163.3483 79.96) (width 0.2) (layer "F.Cu") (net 9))
 (segment (start 163.3483 80.248) (end 162.4846 81.1117) (width 0.2) (layer "F.Cu") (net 9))
 (segment (start 153.2339 81.1117) (end 151.1415 83.2041) (width 0.2) (layer "F.Cu") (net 9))
 (segment (start 163.3483 79.96) (end 163.3483 80.248) (width 0.2) (layer "F.Cu") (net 9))
 (segment (start 151.1415 83.2041) (end 133.0708 83.2041) (width 0.2) (layer "F.Cu") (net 9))
 (segment (start 97.3223 82.7777) (end 96.14 83.96) (width 0.2) (layer "F.Cu") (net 9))
 (segment (start 134 115.04) (end 132.4873 113.5273) (width 0.2) (layer "F.Cu") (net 40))
 (segment (start 132.4873 113.5273) (end 120.2117 113.5273) (width 0.2) (layer "F.Cu") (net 40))
 (via (at 120.2117 113.5273) (size 0.6) (drill 0.3) (layers "F.Cu" "B.Cu") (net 40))
 (segment (start 120.2117 113.5273) (end 119.5909 112.9065) (width 0.2) (layer "B.Cu") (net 40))
 (segment (start 119.5909 112.9065) (end 119.5909 87.0909) (width 0.2) (layer "B.Cu") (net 40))
 (segment (start 119.5909 87.0909) (end 119 86.5) (width 0.2) (layer "B.Cu") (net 40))
 (segment (start 85.98 83.96) (end 87.3683 85.3483) (width 0.2) (layer "F.Cu") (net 23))
 (segment (start 89.79 86.8737) (end 97.0705 94.1542) (width 0.2) (layer "F.Cu") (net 23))
 (segment (start 89.0411 85.3483) (end 89.79 86.0972) (width 0.2) (layer "F.Cu") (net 23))
 (segment (start 134.6542 94.1542) (end 136.5 96) (width 0.2) (layer "F.Cu") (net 23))
 (segment (start 97.0705 94.1542) (end 134.6542 94.1542) (width 0.2) (layer "F.Cu") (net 23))
 (segment (start 89.79 86.0972) (end 89.79 86.8737) (width 0.2) (layer "F.Cu") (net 23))
 (segment (start 87.3683 85.3483) (end 89.0411 85.3483) (width 0.2) (layer "F.Cu") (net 23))
 (segment (start 141.46 79.46) (end 98.1 79.46) (width 0.2) (layer "F.Cu") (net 20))
 (segment (start 98.1 79.46) (end 93.6 83.96) (width 0.2) (layer "F.Cu") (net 20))
 (segment (start 89.79 85.23) (end 88.52 83.96) (width 0.2) (layer "F.Cu") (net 58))
 (segment (start 151.5 88.96) (end 147.77 85.23) (width 0.2) (layer "F.Cu") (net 58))
 (segment (start 147.77 85.23) (end 89.79 85.23) (width 0.2) (layer "F.Cu") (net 58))
 (segment (start 151.123 73.377) (end 154 70.5) (width 0.2) (layer "F.Cu") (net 6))
 (segment (start 91.06 83.96) (end 101.643 73.377) (width 0.2) (layer "F.Cu") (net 6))
 (segment (start 101.643 73.377) (end 151.123 73.377) (width 0.2) (layer "F.Cu") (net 6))
 (segment (start 144 79.46) (end 145.1517 79.46) (width 0.2) (layer "F.Cu") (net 8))
 (segment (start 151.46 79.96) (end 145.6517 79.96) (width 0.2) (layer "F.Cu") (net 8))
 (segment (start 151.46 79.96) (end 151.46 81.896) (width 0.2) (layer "F.Cu") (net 8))
 (segment (start 145.6517 79.96) (end 145.1517 79.46) (width 0.2) (layer "F.Cu") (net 8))
 (segment (start 161.96 79.96) (end 151.46 79.96) (width 0.2) (layer "F.Cu") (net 8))
 (via (at 151.46 81.896) (size 0.6) (drill 0.3) (layers "F.Cu" "B.Cu") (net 8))
 (segment (start 151.46 81.896) (end 151.46 70.5) (width 0.2) (layer "B.Cu") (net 8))
 (segment (start 154.04 88.96) (end 154.04 87.8083) (width 0.2) (layer "B.Cu") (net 8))
 (segment (start 151.46 85.2283) (end 151.46 81.896) (width 0.2) (layer "B.Cu") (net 8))
 (segment (start 154.04 87.8083) (end 151.46 85.2283) (width 0.2) (layer "B.Cu") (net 8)))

